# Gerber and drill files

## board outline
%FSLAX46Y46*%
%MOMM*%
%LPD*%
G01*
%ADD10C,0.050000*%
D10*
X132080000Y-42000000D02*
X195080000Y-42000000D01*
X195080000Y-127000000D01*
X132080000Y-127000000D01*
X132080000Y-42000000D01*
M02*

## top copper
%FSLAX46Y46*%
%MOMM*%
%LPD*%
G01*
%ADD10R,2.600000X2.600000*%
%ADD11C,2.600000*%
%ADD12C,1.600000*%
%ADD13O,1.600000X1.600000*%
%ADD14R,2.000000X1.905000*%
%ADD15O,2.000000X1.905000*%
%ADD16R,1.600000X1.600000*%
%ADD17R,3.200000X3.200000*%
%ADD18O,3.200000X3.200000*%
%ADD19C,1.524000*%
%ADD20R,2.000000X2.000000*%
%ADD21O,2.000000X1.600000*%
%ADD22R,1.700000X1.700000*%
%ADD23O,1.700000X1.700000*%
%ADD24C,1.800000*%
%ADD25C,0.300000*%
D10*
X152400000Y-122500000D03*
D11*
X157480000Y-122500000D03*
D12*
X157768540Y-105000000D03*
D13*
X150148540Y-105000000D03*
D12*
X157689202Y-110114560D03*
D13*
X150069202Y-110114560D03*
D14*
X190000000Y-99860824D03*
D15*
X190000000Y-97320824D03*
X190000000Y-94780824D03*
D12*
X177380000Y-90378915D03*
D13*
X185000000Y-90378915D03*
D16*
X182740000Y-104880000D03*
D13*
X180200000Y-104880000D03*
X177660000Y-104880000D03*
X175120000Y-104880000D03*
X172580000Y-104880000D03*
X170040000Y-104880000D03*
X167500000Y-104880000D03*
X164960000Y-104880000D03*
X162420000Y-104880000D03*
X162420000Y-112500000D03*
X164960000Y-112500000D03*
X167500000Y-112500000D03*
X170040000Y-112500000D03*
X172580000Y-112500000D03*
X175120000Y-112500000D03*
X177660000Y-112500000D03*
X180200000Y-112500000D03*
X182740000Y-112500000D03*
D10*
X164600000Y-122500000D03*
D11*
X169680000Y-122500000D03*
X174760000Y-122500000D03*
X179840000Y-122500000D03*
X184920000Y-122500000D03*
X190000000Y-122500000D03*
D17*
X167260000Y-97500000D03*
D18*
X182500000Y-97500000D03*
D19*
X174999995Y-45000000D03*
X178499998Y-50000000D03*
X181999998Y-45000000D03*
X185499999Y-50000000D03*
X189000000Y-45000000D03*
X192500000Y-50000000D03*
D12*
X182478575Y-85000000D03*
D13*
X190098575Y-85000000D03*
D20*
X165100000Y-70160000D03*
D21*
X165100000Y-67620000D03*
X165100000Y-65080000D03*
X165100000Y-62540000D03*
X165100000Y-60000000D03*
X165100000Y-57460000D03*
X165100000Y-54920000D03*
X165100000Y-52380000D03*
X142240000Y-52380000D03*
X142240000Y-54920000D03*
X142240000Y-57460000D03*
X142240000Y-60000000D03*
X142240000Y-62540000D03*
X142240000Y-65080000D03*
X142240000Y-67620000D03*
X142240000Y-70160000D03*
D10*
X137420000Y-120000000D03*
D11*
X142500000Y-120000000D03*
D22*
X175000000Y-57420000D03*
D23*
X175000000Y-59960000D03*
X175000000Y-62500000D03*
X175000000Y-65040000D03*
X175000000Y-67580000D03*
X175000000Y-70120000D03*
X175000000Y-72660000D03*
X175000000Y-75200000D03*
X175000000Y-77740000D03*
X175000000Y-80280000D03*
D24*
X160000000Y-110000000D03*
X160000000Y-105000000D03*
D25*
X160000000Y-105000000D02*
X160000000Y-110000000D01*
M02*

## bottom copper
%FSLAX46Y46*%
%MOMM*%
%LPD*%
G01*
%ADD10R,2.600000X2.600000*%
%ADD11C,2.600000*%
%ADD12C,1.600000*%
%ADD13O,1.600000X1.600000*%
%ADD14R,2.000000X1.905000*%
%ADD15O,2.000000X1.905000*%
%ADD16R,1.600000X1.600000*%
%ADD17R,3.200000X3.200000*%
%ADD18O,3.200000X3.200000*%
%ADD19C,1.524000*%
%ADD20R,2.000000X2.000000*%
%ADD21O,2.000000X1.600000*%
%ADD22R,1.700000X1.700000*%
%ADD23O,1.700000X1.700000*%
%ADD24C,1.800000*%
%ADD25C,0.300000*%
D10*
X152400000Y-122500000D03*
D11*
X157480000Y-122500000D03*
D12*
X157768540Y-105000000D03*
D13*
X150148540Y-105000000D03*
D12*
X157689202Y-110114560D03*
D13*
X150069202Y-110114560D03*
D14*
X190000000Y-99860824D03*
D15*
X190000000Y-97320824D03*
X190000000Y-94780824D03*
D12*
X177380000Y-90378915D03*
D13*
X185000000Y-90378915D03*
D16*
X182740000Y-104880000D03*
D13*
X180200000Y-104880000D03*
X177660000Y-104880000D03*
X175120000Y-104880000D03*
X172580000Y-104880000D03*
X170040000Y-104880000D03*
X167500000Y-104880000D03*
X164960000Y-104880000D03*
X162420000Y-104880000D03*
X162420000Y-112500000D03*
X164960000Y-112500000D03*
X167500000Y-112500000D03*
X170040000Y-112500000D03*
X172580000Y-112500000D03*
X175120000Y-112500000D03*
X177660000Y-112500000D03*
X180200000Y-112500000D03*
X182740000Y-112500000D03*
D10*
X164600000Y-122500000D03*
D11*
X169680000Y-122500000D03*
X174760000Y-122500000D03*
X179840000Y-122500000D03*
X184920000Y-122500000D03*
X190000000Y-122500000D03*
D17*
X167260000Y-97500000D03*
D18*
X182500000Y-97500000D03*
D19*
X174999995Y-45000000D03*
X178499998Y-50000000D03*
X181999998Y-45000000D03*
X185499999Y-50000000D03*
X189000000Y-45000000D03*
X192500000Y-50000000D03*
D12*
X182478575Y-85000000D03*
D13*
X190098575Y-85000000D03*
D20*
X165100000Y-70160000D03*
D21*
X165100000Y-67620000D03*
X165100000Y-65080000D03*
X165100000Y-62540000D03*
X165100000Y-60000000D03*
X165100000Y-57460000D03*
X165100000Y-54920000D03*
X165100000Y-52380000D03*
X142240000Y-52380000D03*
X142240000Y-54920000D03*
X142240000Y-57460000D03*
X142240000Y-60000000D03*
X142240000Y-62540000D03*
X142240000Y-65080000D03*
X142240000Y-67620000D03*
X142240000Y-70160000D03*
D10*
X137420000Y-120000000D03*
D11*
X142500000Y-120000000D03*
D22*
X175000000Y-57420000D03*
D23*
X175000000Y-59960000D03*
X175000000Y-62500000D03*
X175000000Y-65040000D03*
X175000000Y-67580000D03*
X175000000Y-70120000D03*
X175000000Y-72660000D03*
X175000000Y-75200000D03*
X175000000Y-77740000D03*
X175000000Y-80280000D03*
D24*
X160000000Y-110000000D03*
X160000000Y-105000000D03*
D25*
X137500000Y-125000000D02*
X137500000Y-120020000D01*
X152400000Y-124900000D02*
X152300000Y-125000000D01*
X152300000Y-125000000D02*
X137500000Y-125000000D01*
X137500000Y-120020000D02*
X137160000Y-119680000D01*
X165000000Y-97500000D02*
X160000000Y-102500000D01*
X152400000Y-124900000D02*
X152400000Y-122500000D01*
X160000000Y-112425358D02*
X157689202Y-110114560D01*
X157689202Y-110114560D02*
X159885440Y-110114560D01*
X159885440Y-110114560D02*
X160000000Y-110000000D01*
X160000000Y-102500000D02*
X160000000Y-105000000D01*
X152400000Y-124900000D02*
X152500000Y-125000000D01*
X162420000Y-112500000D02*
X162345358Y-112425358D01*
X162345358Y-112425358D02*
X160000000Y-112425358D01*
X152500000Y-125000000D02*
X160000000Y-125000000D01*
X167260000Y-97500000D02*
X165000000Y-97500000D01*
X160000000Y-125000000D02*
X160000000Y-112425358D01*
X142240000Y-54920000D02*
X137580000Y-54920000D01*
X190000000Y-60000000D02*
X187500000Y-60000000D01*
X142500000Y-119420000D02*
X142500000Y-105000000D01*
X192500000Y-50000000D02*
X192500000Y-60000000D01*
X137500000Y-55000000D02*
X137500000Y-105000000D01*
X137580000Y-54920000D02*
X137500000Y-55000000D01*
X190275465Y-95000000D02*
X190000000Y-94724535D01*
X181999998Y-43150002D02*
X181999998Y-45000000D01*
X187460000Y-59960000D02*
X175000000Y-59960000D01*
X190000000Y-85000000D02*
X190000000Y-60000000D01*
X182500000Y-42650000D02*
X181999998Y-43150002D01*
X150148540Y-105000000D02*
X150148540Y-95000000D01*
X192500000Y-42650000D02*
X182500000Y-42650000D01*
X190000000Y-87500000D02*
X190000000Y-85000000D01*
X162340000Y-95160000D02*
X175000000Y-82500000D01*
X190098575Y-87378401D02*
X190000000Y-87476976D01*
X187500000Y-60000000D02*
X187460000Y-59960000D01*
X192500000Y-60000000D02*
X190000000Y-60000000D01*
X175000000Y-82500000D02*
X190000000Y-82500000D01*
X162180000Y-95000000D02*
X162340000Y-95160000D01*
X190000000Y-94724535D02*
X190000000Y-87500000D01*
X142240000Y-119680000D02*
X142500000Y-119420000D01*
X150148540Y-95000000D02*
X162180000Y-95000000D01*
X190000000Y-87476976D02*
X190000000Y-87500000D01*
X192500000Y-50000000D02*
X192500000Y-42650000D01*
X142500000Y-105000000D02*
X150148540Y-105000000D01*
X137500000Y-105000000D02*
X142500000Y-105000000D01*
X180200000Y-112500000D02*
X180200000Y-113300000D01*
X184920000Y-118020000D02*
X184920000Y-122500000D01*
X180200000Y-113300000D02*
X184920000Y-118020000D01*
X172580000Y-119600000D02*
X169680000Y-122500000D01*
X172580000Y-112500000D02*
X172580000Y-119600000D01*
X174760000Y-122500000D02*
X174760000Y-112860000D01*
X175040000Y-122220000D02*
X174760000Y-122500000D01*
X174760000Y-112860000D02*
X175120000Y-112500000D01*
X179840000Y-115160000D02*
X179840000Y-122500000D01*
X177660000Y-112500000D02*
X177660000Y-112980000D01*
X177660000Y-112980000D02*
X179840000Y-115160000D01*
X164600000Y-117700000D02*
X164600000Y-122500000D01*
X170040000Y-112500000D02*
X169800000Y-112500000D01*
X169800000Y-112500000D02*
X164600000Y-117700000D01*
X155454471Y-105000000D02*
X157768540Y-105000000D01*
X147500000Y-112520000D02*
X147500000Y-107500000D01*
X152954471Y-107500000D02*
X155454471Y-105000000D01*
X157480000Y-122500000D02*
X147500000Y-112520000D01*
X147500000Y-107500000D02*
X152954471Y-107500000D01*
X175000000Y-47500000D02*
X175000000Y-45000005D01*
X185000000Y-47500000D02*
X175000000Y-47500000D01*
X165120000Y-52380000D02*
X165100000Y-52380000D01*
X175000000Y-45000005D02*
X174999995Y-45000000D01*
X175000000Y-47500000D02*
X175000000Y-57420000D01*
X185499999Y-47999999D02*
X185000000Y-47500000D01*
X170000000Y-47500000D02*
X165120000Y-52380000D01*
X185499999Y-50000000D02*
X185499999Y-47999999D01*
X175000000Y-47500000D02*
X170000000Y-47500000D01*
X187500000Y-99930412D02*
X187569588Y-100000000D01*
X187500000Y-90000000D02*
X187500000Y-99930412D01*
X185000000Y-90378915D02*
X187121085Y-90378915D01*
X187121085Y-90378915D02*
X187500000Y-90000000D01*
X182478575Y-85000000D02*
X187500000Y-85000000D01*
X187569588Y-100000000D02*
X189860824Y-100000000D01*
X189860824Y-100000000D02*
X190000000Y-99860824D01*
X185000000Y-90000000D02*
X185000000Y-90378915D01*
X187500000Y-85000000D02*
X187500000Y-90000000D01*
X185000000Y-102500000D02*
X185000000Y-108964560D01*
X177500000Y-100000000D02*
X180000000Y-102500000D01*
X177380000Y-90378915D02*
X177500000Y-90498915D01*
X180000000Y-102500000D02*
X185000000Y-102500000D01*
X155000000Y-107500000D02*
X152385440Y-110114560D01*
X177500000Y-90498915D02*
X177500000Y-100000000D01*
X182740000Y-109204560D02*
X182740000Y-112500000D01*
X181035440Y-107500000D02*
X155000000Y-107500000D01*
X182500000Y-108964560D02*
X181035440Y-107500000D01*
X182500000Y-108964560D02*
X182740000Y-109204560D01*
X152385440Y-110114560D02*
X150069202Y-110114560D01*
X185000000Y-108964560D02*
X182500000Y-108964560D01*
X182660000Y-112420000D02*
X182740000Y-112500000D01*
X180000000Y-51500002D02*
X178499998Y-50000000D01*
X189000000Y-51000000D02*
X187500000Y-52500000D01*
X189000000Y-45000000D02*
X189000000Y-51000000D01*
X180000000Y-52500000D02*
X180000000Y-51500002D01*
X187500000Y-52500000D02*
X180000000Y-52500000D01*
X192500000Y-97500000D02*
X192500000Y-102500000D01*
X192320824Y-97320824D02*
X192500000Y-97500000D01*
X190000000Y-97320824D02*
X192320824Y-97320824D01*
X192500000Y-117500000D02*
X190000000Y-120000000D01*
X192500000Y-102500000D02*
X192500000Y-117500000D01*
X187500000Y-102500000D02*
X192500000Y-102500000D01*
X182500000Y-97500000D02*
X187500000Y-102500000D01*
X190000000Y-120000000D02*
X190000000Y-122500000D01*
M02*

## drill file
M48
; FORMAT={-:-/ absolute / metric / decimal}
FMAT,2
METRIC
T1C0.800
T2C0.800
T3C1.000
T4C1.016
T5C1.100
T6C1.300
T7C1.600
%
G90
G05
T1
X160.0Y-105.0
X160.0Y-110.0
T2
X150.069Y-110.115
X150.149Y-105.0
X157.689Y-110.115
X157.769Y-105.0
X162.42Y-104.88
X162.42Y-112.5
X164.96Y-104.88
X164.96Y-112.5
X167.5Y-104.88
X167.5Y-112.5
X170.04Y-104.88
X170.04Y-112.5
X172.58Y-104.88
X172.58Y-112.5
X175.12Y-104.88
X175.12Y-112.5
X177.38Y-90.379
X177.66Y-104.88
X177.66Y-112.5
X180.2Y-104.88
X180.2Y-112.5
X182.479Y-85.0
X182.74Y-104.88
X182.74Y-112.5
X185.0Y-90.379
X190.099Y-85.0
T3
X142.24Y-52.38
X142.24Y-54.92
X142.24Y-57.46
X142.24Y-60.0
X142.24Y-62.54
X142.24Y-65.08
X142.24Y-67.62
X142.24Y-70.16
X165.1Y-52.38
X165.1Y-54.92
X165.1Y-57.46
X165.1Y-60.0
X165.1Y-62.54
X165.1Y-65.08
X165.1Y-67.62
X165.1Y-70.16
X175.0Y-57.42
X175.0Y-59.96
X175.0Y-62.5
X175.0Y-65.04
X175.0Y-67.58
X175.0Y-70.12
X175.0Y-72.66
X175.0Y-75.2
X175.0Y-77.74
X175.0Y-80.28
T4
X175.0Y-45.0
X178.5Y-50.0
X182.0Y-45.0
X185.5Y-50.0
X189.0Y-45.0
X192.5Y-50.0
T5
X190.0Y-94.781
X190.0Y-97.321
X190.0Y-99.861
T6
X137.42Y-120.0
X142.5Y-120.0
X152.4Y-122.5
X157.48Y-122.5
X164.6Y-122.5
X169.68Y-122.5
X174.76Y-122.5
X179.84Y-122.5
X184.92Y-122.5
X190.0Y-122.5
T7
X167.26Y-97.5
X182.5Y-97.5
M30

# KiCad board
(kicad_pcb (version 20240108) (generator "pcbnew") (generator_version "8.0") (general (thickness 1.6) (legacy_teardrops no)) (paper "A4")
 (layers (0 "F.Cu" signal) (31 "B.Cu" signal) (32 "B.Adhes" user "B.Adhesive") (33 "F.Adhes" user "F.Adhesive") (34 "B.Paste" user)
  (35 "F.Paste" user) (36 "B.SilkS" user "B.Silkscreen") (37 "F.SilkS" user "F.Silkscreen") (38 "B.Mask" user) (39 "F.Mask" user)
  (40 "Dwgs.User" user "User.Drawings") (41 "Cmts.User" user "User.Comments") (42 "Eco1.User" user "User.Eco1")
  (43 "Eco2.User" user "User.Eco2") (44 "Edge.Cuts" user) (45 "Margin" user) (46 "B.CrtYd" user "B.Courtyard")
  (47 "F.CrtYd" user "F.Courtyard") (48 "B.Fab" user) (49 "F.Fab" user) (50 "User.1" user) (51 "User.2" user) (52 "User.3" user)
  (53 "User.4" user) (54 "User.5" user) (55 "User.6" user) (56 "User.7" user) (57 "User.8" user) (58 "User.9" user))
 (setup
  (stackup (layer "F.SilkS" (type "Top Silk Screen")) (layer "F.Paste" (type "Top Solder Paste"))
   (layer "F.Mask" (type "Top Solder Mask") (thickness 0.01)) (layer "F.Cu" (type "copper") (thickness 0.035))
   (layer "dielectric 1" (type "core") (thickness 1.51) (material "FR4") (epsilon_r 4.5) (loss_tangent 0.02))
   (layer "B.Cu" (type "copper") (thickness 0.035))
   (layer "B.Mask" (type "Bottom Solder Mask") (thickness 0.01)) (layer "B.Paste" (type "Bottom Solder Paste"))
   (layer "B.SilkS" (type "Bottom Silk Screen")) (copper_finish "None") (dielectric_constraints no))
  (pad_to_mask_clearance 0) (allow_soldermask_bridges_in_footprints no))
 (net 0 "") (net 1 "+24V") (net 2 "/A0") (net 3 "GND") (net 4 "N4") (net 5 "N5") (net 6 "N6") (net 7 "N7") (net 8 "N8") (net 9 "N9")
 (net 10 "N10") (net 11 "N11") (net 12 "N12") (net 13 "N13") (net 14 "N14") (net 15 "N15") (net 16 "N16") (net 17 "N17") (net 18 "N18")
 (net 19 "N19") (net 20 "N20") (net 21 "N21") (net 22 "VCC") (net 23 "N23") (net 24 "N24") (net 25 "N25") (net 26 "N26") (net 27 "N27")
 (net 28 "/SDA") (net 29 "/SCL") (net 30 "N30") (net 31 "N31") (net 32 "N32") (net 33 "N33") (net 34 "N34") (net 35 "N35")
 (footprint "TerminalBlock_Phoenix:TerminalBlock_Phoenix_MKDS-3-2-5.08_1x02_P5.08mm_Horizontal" (layer "F.Cu") (at 152.4 122.5)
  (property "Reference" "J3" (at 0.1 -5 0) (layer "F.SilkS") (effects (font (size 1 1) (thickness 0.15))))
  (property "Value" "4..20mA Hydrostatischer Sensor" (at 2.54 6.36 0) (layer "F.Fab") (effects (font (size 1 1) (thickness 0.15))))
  (pad "1" thru_hole rect (at 0 0) (size 2.6 2.6) (drill 1.3) (layers "*.Cu" "*.Mask") (remove_unused_layers no) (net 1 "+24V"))
  (pad "2" thru_hole circle (at 5.08 0) (size 2.6 2.6) (drill 1.3) (layers "*.Cu" "*.Mask") (remove_unused_layers no) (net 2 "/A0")))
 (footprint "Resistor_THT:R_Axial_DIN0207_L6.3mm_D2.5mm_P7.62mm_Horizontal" (layer "F.Cu") (at 157.76854 105 180)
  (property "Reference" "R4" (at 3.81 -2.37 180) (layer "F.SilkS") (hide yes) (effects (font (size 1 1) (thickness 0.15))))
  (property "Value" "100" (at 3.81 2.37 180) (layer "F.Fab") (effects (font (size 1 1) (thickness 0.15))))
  (pad "1" thru_hole circle (at 0 0 180) (size 1.6 1.6) (drill 0.8) (layers "*.Cu" "*.Mask") (remove_unused_layers no) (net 2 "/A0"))
  (pad "2" thru_hole oval (at 7.62 0 180) (size 1.6 1.6) (drill 0.8) (layers "*.Cu" "*.Mask") (remove_unused_layers no) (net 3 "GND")))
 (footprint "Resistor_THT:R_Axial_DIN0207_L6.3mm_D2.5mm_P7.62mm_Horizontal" (layer "F.Cu") (at 157.689202 110.11456 180)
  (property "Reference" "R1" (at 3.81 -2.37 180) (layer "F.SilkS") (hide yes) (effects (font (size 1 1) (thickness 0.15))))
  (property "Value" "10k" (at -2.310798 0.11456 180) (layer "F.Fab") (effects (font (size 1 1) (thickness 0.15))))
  (pad "1" thru_hole circle (at 0 0 180) (size 1.6 1.6) (drill 0.8) (layers "*.Cu" "*.Mask") (remove_unused_layers no) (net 1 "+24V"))
  (pad "2" thru_hole oval (at 7.62 0 180) (size 1.6 1.6) (drill 0.8) (layers "*.Cu" "*.Mask") (remove_unused_layers no) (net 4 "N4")))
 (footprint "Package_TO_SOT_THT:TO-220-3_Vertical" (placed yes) (layer "F.Cu") (at 190 99.860824 90)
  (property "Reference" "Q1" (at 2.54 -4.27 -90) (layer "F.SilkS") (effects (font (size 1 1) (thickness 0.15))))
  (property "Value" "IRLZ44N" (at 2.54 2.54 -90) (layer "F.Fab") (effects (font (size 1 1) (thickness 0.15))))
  (pad "1" thru_hole rect (at 0 0 90) (size 1.905 2) (drill 1.1) (layers "*.Cu" "*.Mask") (remove_unused_layers no) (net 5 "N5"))
  (pad "2" thru_hole oval (at 2.54 0 90) (size 1.905 2) (drill 1.1) (layers "*.Cu" "*.Mask") (remove_unused_layers no) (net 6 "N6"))
  (pad "3" thru_hole oval (at 5.08 0 90) (size 1.905 2) (drill 1.1) (layers "*.Cu" "*.Mask") (remove_unused_layers no) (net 3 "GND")))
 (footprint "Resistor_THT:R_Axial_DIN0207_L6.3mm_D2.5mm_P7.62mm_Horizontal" (layer "F.Cu") (at 177.38 90.378915)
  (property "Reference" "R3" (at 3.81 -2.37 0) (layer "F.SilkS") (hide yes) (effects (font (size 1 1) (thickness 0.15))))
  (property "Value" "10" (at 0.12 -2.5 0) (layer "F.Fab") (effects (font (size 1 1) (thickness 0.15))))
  (pad "1" thru_hole circle (at 0 0) (size 1.6 1.6) (drill 0.8) (layers "*.Cu" "*.Mask") (remove_unused_layers no) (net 4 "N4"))
  (pad "2" thru_hole oval (at 7.62 0) (size 1.6 1.6) (drill 0.8) (layers "*.Cu" "*.Mask") (remove_unused_layers no) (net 5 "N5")))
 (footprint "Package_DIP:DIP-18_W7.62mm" (layer "F.Cu") (at 182.74 104.88 -90)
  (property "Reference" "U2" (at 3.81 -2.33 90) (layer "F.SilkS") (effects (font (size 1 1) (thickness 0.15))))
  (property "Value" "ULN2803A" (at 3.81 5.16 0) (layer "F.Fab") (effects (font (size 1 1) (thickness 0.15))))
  (pad "1" thru_hole rect (at 0 0 270) (size 1.6 1.6) (drill 0.8) (layers "*.Cu" "*.Mask") (remove_unused_layers no) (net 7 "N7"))
  (pad "2" thru_hole oval (at 0 2.54 270) (size 1.6 1.6) (drill 0.8) (layers "*.Cu" "*.Mask") (remove_unused_layers no) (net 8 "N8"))
  (pad "3" thru_hole oval (at 0 5.08 270) (size 1.6 1.6) (drill 0.8) (layers "*.Cu" "*.Mask") (remove_unused_layers no) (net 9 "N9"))
  (pad "4" thru_hole oval (at 0 7.62 270) (size 1.6 1.6) (drill 0.8) (layers "*.Cu" "*.Mask") (remove_unused_layers no) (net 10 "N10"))
  (pad "5" thru_hole oval (at 0 10.16 270) (size 1.6 1.6) (drill 0.8) (layers "*.Cu" "*.Mask") (remove_unused_layers no) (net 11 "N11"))
  (pad "6" thru_hole oval (at 0 12.7 270) (size 1.6 1.6) (drill 0.8) (layers "*.Cu" "*.Mask") (remove_unused_layers no) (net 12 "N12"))
  (pad "7" thru_hole oval (at 0 15.24 270) (size 1.6 1.6) (drill 0.8) (layers "*.Cu" "*.Mask") (remove_unused_layers no) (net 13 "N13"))
  (pad "8" thru_hole oval (at 0 17.78 270) (size 1.6 1.6) (drill 0.8) (layers "*.Cu" "*.Mask") (remove_unused_layers no) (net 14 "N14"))
  (pad "9" thru_hole oval (at 0 20.32 270) (size 1.6 1.6) (drill 0.8) (layers "*.Cu" "*.Mask") (remove_unused_layers no) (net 3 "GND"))
  (pad "10" thru_hole oval (at 7.62 20.32 270) (size 1.6 1.6) (drill 0.8) (layers "*.Cu" "*.Mask") (remove_unused_layers no) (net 1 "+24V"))
  (pad "11" thru_hole oval (at 7.62 17.78 270) (size 1.6 1.6) (drill 0.8) (layers "*.Cu" "*.Mask") (remove_unused_layers no) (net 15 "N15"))
  (pad "12" thru_hole oval (at 7.62 15.24 270) (size 1.6 1.6) (drill 0.8) (layers "*.Cu" "*.Mask") (remove_unused_layers no) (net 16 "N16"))
  (pad "13" thru_hole oval (at 7.62 12.7 270) (size 1.6 1.6) (drill 0.8) (layers "*.Cu" "*.Mask") (remove_unused_layers no) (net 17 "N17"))
  (pad "14" thru_hole oval (at 7.62 10.16 270) (size 1.6 1.6) (drill 0.8) (layers "*.Cu" "*.Mask") (remove_unused_layers no) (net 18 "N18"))
  (pad "15" thru_hole oval (at 7.62 7.62 270) (size 1.6 1.6) (drill 0.8) (layers "*.Cu" "*.Mask") (remove_unused_layers no) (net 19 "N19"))
  (pad "16" thru_hole oval (at 7.62 5.08 270) (size 1.6 1.6) (drill 0.8) (layers "*.Cu" "*.Mask") (remove_unused_layers no) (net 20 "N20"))
  (pad "17" thru_hole oval (at 7.62 2.54 270) (size 1.6 1.6) (drill 0.8) (layers "*.Cu" "*.Mask") (remove_unused_layers no) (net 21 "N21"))
  (pad "18" thru_hole oval (at 7.62 0 270) (size 1.6 1.6) (drill 0.8) (layers "*.Cu" "*.Mask") (remove_unused_layers no) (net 4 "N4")))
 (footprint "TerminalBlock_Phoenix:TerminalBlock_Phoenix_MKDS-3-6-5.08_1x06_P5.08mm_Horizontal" (layer "F.Cu") (at 164.6 122.5)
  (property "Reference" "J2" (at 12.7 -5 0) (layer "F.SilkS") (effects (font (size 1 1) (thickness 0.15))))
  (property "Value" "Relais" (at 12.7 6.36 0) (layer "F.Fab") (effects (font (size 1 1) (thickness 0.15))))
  (pad "1" thru_hole rect (at 0 0) (size 2.6 2.6) (drill 1.3) (layers "*.Cu" "*.Mask") (remove_unused_layers no) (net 17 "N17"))
  (pad "2" thru_hole circle (at 5.08 0) (size 2.6 2.6) (drill 1.3) (layers "*.Cu" "*.Mask") (remove_unused_layers no) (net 18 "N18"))
  (pad "3" thru_hole circle (at 10.16 0) (size 2.6 2.6) (drill 1.3) (layers "*.Cu" "*.Mask") (remove_unused_layers no) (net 19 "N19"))
  (pad "4" thru_hole circle (at 15.24 0) (size 2.6 2.6) (drill 1.3) (layers "*.Cu" "*.Mask") (remove_unused_layers no) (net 20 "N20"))
  (pad "5" thru_hole circle (at 20.32 0) (size 2.6 2.6) (drill 1.3) (layers "*.Cu" "*.Mask") (remove_unused_layers no) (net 21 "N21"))
  (pad "6" thru_hole circle (at 25.4 0) (size 2.6 2.6) (drill 1.3) (layers "*.Cu" "*.Mask") (remove_unused_layers no) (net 6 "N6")))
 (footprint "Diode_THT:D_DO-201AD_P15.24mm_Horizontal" (layer "F.Cu") (at 167.26 97.5)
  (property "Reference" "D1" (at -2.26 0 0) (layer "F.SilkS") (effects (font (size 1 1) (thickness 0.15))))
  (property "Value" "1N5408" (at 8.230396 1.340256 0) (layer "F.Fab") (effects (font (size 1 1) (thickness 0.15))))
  (pad "1" thru_hole rect (at 0 0) (size 3.2 3.2) (drill 1.6) (layers "*.Cu" "*.Mask") (remove_unused_layers no) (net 1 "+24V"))
  (pad "2" thru_hole oval (at 15.24 0) (size 3.2 3.2) (drill 1.6) (layers "*.Cu" "*.Mask") (remove_unused_layers no) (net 6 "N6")))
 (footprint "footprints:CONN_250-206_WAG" (layer "F.Cu") (at 174.999995 45)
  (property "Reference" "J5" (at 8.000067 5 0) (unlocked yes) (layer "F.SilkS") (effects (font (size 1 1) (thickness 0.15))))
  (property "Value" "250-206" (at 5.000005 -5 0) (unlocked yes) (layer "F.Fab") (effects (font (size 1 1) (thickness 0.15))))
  (pad "1" thru_hole circle (at 0 0) (size 1.524 1.524) (drill 1.016) (layers "*.Cu" "*.Mask") (remove_unused_layers no) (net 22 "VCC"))
  (pad "2" thru_hole circle (at 3.500003 5) (size 1.524 1.524) (drill 1.016) (layers "*.Cu" "*.Mask") (remove_unused_layers no)
   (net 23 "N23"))
  (pad "3" thru_hole circle (at 7.000003 0) (size 1.524 1.524) (drill 1.016) (layers "*.Cu" "*.Mask") (remove_unused_layers no)
   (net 3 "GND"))
  (pad "4" thru_hole circle (at 10.500004 5) (size 1.524 1.524) (drill 1.016) (layers "*.Cu" "*.Mask") (remove_unused_layers no)
   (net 22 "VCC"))
  (pad "5" thru_hole circle (at 14.000005 0) (size 1.524 1.524) (drill 1.016) (layers "*.Cu" "*.Mask") (remove_unused_layers no)
   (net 23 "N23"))
  (pad "6" thru_hole circle (at 17.500005 5) (size 1.524 1.524) (drill 1.016) (layers "*.Cu" "*.Mask") (remove_unused_layers no)
   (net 3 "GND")))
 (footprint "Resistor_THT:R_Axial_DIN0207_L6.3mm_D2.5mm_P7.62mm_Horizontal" (layer "F.Cu") (at 182.478575 85)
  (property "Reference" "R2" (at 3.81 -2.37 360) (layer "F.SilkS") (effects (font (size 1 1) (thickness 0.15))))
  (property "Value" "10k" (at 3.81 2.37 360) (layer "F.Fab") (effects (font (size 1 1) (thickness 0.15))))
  (pad "1" thru_hole circle (at 0 0) (size 1.6 1.6) (drill 0.8) (layers "*.Cu" "*.Mask") (remove_unused_layers no) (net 5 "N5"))
  (pad "2" thru_hole oval (at 7.62 0) (size 1.6 1.6) (drill 0.8) (layers "*.Cu" "*.Mask") (remove_unused_layers no) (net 3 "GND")))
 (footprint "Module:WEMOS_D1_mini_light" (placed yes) (layer "F.Cu") (at 165.1 70.16 180)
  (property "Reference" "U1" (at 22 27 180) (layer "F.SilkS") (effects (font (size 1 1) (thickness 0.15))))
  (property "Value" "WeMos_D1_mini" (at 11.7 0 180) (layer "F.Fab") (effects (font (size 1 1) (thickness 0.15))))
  (pad "1" thru_hole rect (at 0 0 180) (size 2 2) (drill 1) (layers "*.Cu" "*.Mask") (remove_unused_layers no) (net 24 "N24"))
  (pad "2" thru_hole oval (at 0 2.54 180) (size 2 1.6) (drill 1) (layers "*.Cu" "*.Mask") (remove_unused_layers no) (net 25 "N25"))
  (pad "3" thru_hole oval (at 0 5.08 180) (size 2 1.6) (drill 1) (layers "*.Cu" "*.Mask") (remove_unused_layers no) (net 7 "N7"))
  (pad "4" thru_hole oval (at 0 7.62 180) (size 2 1.6) (drill 1) (layers "*.Cu" "*.Mask") (remove_unused_layers no) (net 11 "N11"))
  (pad "5" thru_hole oval (at 0 10.16 180) (size 2 1.6) (drill 1) (layers "*.Cu" "*.Mask") (remove_unused_layers no) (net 9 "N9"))
  (pad "6" thru_hole oval (at 0 12.7 180) (size 2 1.6) (drill 1) (layers "*.Cu" "*.Mask") (remove_unused_layers no) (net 10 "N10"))
  (pad "7" thru_hole oval (at 0 15.24 180) (size 2 1.6) (drill 1) (layers "*.Cu" "*.Mask") (remove_unused_layers no) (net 12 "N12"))
  (pad "8" thru_hole oval (at 0 17.78 180) (size 2 1.6) (drill 1) (layers "*.Cu" "*.Mask") (remove_unused_layers no) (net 22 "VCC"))
  (pad "9" thru_hole oval (at 22.86 17.78 180) (size 2 1.6) (drill 1) (layers "*.Cu" "*.Mask") (remove_unused_layers no) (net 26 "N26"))
  (pad "10" thru_hole oval (at 22.86 15.24 180) (size 2 1.6) (drill 1) (layers "*.Cu" "*.Mask") (remove_unused_layers no) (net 3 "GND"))
  (pad "11" thru_hole oval (at 22.86 12.7 180) (size 2 1.6) (drill 1) (layers "*.Cu" "*.Mask") (remove_unused_layers no) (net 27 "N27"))
  (pad "12" thru_hole oval (at 22.86 10.16 180) (size 2 1.6) (drill 1) (layers "*.Cu" "*.Mask") (remove_unused_layers no) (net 23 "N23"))
  (pad "13" thru_hole oval (at 22.86 7.62 180) (size 2 1.6) (drill 1) (layers "*.Cu" "*.Mask") (remove_unused_layers no) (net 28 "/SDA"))
  (pad "14" thru_hole oval (at 22.86 5.08 180) (size 2 1.6) (drill 1) (layers "*.Cu" "*.Mask") (remove_unused_layers no) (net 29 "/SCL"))
  (pad "15" thru_hole oval (at 22.86 2.54 180) (size 2 1.6) (drill 1) (layers "*.Cu" "*.Mask") (remove_unused_layers no) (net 8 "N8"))
  (pad "16" thru_hole oval (at 22.86 0 180) (size 2 1.6) (drill 1) (layers "*.Cu" "*.Mask") (remove_unused_layers no) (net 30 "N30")))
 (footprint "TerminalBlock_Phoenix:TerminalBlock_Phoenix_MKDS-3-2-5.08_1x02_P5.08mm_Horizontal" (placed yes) (layer "F.Cu") (at 137.42 120)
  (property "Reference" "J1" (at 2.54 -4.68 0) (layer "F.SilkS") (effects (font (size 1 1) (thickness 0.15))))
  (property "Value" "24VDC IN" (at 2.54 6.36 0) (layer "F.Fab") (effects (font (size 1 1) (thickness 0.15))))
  (pad "1" thru_hole rect (at 0 0) (size 2.6 2.6) (drill 1.3) (layers "*.Cu" "*.Mask") (remove_unused_layers no) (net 1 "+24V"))
  (pad "2" thru_hole circle (at 5.08 0) (size 2.6 2.6) (drill 1.3) (layers "*.Cu" "*.Mask") (remove_unused_layers no) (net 3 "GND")))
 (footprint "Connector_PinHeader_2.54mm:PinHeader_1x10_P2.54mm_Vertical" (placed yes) (layer "F.Cu") (at 175 57.42)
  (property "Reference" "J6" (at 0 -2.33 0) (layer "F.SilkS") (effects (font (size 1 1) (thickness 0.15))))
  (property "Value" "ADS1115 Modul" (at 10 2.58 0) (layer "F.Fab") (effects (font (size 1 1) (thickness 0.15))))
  (pad "1" thru_hole rect (at 0 0) (size 1.7 1.7) (drill 1) (layers "*.Cu" "*.Mask") (remove_unused_layers no) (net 22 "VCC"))
  (pad "2" thru_hole oval (at 0 2.54) (size 1.7 1.7) (drill 1) (layers "*.Cu" "*.Mask") (remove_unused_layers no) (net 3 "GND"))
  (pad "3" thru_hole oval (at 0 5.08) (size 1.7 1.7) (drill 1) (layers "*.Cu" "*.Mask") (remove_unused_layers no) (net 29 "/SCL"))
  (pad "4" thru_hole oval (at 0 7.62) (size 1.7 1.7) (drill 1) (layers "*.Cu" "*.Mask") (remove_unused_layers no) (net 28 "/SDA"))
  (pad "5" thru_hole oval (at 0 10.16) (size 1.7 1.7) (drill 1) (layers "*.Cu" "*.Mask") (remove_unused_layers no) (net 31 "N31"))
  (pad "6" thru_hole oval (at 0 12.7) (size 1.7 1.7) (drill 1) (layers "*.Cu" "*.Mask") (remove_unused_layers no) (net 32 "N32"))
  (pad "7" thru_hole oval (at 0 15.24) (size 1.7 1.7) (drill 1) (layers "*.Cu" "*.Mask") (remove_unused_layers no) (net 2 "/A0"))
  (pad "8" thru_hole oval (at 0 17.78) (size 1.7 1.7) (drill 1) (layers "*.Cu" "*.Mask") (remove_unused_layers no) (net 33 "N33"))
  (pad "9" thru_hole oval (at 0 20.32) (size 1.7 1.7) (drill 1) (layers "*.Cu" "*.Mask") (remove_unused_layers no) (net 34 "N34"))
  (pad "10" thru_hole oval (at 0 22.86) (size 1.7 1.7) (drill 1) (layers "*.Cu" "*.Mask") (remove_unused_layers no) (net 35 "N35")))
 (gr_rect (start 132.08 42) (end 195.08 127) (stroke (width 0.05) (type default)) (fill none) (layer "Edge.Cuts"))
 (segment (start 160 105) (end 160 110) (width 0.3) (layer "F.Cu") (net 1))
 (via (at 160 110) (size 1.8) (drill 0.8) (layers "F.Cu" "B.Cu") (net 1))
 (via (at 160 105) (size 1.8) (drill 0.8) (layers "F.Cu" "B.Cu") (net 1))
 (segment (start 137.5 125) (end 137.5 120.02) (width 0.3) (layer "B.Cu") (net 1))
 (segment (start 152.4 124.9) (end 152.3 125) (width 0.3) (layer "B.Cu") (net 1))
 (segment (start 152.3 125) (end 137.5 125) (width 0.3) (layer "B.Cu") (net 1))
 (segment (start 137.5 120.02) (end 137.16 119.68) (width 0.3) (layer "B.Cu") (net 1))
 (segment (start 165 97.5) (end 160 102.5) (width 0.3) (layer "B.Cu") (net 1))
 (segment (start 152.4 124.9) (end 152.4 122.5) (width 0.3) (layer "B.Cu") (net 1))
 (segment (start 160 112.425358) (end 157.689202 110.11456) (width 0.3) (layer "B.Cu") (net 1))
 (segment (start 157.689202 110.11456) (end 159.88544 110.11456) (width 0.3) (layer "B.Cu") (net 1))
 (segment (start 159.88544 110.11456) (end 160 110) (width 0.3) (layer "B.Cu") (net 1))
 (segment (start 160 102.5) (end 160 105) (width 0.3) (layer "B.Cu") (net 1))
 (segment (start 152.4 124.9) (end 152.5 125) (width 0.3) (layer "B.Cu") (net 1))
 (segment (start 162.42 112.5) (end 162.345358 112.425358) (width 0.3) (layer "B.Cu") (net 1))
 (segment (start 162.345358 112.425358) (end 160 112.425358) (width 0.3) (layer "B.Cu") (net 1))
 (segment (start 152.5 125) (end 160 125) (width 0.3) (layer "B.Cu") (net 1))
 (segment (start 167.26 97.5) (end 165 97.5) (width 0.3) (layer "B.Cu") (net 1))
 (segment (start 160 125) (end 160 112.425358) (width 0.3) (layer "B.Cu") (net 1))
 (segment (start 142.24 54.92) (end 137.58 54.92) (width 0.3) (layer "B.Cu") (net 3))
 (segment (start 190 60) (end 187.5 60) (width 0.3) (layer "B.Cu") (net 3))
 (segment (start 142.5 119.42) (end 142.5 105) (width 0.3) (layer "B.Cu") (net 3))
 (segment (start 192.5 50) (end 192.5 60) (width 0.3) (layer "B.Cu") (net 3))
 (segment (start 137.5 55) (end 137.5 105) (width 0.3) (layer "B.Cu") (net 3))
 (segment (start 137.58 54.92) (end 137.5 55) (width 0.3) (layer "B.Cu") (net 3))
 (segment (start 190.275465 95) (end 190 94.724535) (width 0.3) (layer "B.Cu") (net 3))
 (segment (start 181.999998 43.150002) (end 181.999998 45) (width 0.3) (layer "B.Cu") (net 3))
 (segment (start 187.46 59.96) (end 175 59.96) (width 0.3) (layer "B.Cu") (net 3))
 (segment (start 190 85) (end 190 60) (width 0.3) (layer "B.Cu") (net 3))
 (segment (start 182.5 42.65) (end 181.999998 43.150002) (width 0.3) (layer "B.Cu") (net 3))
 (segment (start 150.14854 105) (end 150.14854 95) (width 0.3) (layer "B.Cu") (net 3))
 (segment (start 192.5 42.65) (end 182.5 42.65) (width 0.3) (layer "B.Cu") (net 3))
 (segment (start 190 87.5) (end 190 85) (width 0.3) (layer "B.Cu") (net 3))
 (segment (start 162.34 95.16) (end 175 82.5) (width 0.3) (layer "B.Cu") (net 3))
 (segment (start 190.098575 87.378401) (end 190 87.476976) (width 0.3) (layer "B.Cu") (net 3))
 (segment (start 187.5 60) (end 187.46 59.96) (width 0.3) (layer "B.Cu") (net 3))
 (segment (start 192.5 60) (end 190 60) (width 0.3) (layer "B.Cu") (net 3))
 (segment (start 175 82.5) (end 190 82.5) (width 0.3) (layer "B.Cu") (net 3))
 (segment (start 162.18 95) (end 162.34 95.16) (width 0.3) (layer "B.Cu") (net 3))
 (segment (start 190 94.724535) (end 190 87.5) (width 0.3) (layer "B.Cu") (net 3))
 (segment (start 142.24 119.68) (end 142.5 119.42) (width 0.3) (layer "B.Cu") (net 3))
 (segment (start 150.14854 95) (end 162.18 95) (width 0.3) (layer "B.Cu") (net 3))
 (segment (start 190 87.476976) (end 190 87.5) (width 0.3) (layer "B.Cu") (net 3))
 (segment (start 192.5 50) (end 192.5 42.65) (width 0.3) (layer "B.Cu") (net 3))
 (segment (start 142.5 105) (end 150.14854 105) (width 0.3) (layer "B.Cu") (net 3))
 (segment (start 137.5 105) (end 142.5 105) (width 0.3) (layer "B.Cu") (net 3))
 (segment (start 180.2 112.5) (end 180.2 113.3) (width 0.3) (layer "B.Cu") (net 21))
 (segment (start 184.92 118.02) (end 184.92 122.5) (width 0.3) (layer "B.Cu") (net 21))
 (segment (start 180.2 113.3) (end 184.92 118.02) (width 0.3) (layer "B.Cu") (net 21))
 (segment (start 172.58 119.6) (end 169.68 122.5) (width 0.3) (layer "B.Cu") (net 18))
 (segment (start 172.58 112.5) (end 172.58 119.6) (width 0.3) (layer "B.Cu") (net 18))
 (segment (start 174.76 122.5) (end 174.76 112.86) (width 0.3) (layer "B.Cu") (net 19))
 (segment (start 175.04 122.22) (end 174.76 122.5) (width 0.3) (layer "B.Cu") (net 19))
 (segment (start 174.76 112.86) (end 175.12 112.5) (width 0.3) (layer "B.Cu") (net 19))
 (segment (start 179.84 115.16) (end 179.84 122.5) (width 0.3) (layer "B.Cu") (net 20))
 (segment (start 177.66 112.5) (end 177.66 112.98) (width 0.3) (layer "B.Cu") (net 20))
 (segment (start 177.66 112.98) (end 179.84 115.16) (width 0.3) (layer "B.Cu") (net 20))
 (segment (start 164.6 117.7) (end 164.6 122.5) (width 0.3) (layer "B.Cu") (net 17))
 (segment (start 170.04 112.5) (end 169.8 112.5) (width 0.3) (layer "B.Cu") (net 17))
 (segment (start 169.8 112.5) (end 164.6 117.7) (width 0.3) (layer "B.Cu") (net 17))
 (segment (start 155.454471 105) (end 157.76854 105) (width 0.3) (layer "B.Cu") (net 2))
 (segment (start 147.5 112.52) (end 147.5 107.5) (width 0.3) (layer "B.Cu") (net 2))
 (segment (start 152.954471 107.5) (end 155.454471 105) (width 0.3) (layer "B.Cu") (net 2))
 (segment (start 157.48 122.5) (end 147.5 112.52) (width 0.3) (layer "B.Cu") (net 2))
 (segment (start 147.5 107.5) (end 152.954471 107.5) (width 0.3) (layer "B.Cu") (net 2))
 (segment (start 175 47.5) (end 175 45.000005) (width 0.3) (layer "B.Cu") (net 22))
 (segment (start 185 47.5) (end 175 47.5) (width 0.3) (layer "B.Cu") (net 22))
 (segment (start 165.12 52.38) (end 165.1 52.38) (width 0.3) (layer "B.Cu") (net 22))
 (segment (start 175 45.000005) (end 174.999995 45) (width 0.3) (layer "B.Cu") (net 22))
 (segment (start 175 47.5) (end 175 57.42) (width 0.3) (layer "B.Cu") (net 22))
 (segment (start 185.499999 47.999999) (end 185 47.5) (width 0.3) (layer "B.Cu") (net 22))
 (segment (start 170 47.5) (end 165.12 52.38) (width 0.3) (layer "B.Cu") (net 22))
 (segment (start 185.499999 50) (end 185.499999 47.999999) (width 0.3) (layer "B.Cu") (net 22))
 (segment (start 175 47.5) (end 170 47.5) (width 0.3) (layer "B.Cu") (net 22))
 (segment (start 187.5 99.930412) (end 187.569588 100) (width 0.3) (layer "B.Cu") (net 5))
 (segment (start 187.5 90) (end 187.5 99.930412) (width 0.3) (layer "B.Cu") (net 5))
 (segment (start 185 90.378915) (end 187.121085 90.378915) (width 0.3) (layer "B.Cu") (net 5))
 (segment (start 187.121085 90.378915) (end 187.5 90) (width 0.3) (layer "B.Cu") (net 5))
 (segment (start 182.478575 85) (end 187.5 85) (width 0.3) (layer "B.Cu") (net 5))
 (segment (start 187.569588 100) (end 189.860824 100) (width 0.3) (layer "B.Cu") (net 5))
 (segment (start 189.860824 100) (end 190 99.860824) (width 0.3) (layer "B.Cu") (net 5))
 (segment (start 185 90) (end 185 90.378915) (width 0.3) (layer "B.Cu") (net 5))
 (segment (start 187.5 85) (end 187.5 90) (width 0.3) (layer "B.Cu") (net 5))
 (segment (start 185 102.5) (end 185 108.96456) (width 0.3) (layer "B.Cu") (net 4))
 (segment (start 177.5 100) (end 180 102.5) (width 0.3) (layer "B.Cu") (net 4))
 (segment (start 177.38 90.378915) (end 177.5 90.498915) (width 0.3) (layer "B.Cu") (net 4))
 (segment (start 180 102.5) (end 185 102.5) (width 0.3) (layer "B.Cu") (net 4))
 (segment (start 155 107.5) (end 152.38544 110.11456) (width 0.3) (layer "B.Cu") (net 4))
 (segment (start 177.5 90.498915) (end 177.5 100) (width 0.3) (layer "B.Cu") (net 4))
 (segment (start 182.74 109.20456) (end 182.74 112.5) (width 0.3) (layer "B.Cu") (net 4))
 (segment (start 181.03544 107.5) (end 155 107.5) (width 0.3) (layer "B.Cu") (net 4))
 (segment (start 182.5 108.96456) (end 181.03544 107.5) (width 0.3) (layer "B.Cu") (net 4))
 (segment (start 182.5 108.96456) (end 182.74 109.20456) (width 0.3) (layer "B.Cu") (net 4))
 (segment (start 152.38544 110.11456) (end 150.069202 110.11456) (width 0.3) (layer "B.Cu") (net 4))
 (segment (start 185 108.96456) (end 182.5 108.96456) (width 0.3) (layer "B.Cu") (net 4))
 (segment (start 182.66 112.42) (end 182.74 112.5) (width 0.3) (layer "B.Cu") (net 4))
 (segment (start 180 51.500002) (end 178.499998 50) (width 0.3) (layer "B.Cu") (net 23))
 (segment (start 189 51) (end 187.5 52.5) (width 0.3) (layer "B.Cu") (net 23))
 (segment (start 189 45) (end 189 51) (width 0.3) (layer "B.Cu") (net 23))
 (segment (start 180 52.5) (end 180 51.500002) (width 0.3) (layer "B.Cu") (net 23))
 (segment (start 187.5 52.5) (end 180 52.5) (width 0.3) (layer "B.Cu") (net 23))
 (segment (start 192.5 97.5) (end 192.5 102.5) (width 0.3) (layer "B.Cu") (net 6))
 (segment (start 192.320824 97.320824) (end 192.5 97.5) (width 0.3) (layer "B.Cu") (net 6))
 (segment (start 190 97.320824) (end 192.320824 97.320824) (width 0.3) (layer "B.Cu") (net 6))
 (segment (start 192.5 117.5) (end 190 120) (width 0.3) (layer "B.Cu") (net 6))
 (segment (start 192.5 102.5) (end 192.5 117.5) (width 0.3) (layer "B.Cu") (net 6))
 (segment (start 187.5 102.5) (end 192.5 102.5) (width 0.3) (layer "B.Cu") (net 6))
 (segment (start 182.5 97.5) (end 187.5 102.5) (width 0.3) (layer "B.Cu") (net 6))
 (segment (start 190 120) (end 190 122.5) (width 0.3) (layer "B.Cu") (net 6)))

